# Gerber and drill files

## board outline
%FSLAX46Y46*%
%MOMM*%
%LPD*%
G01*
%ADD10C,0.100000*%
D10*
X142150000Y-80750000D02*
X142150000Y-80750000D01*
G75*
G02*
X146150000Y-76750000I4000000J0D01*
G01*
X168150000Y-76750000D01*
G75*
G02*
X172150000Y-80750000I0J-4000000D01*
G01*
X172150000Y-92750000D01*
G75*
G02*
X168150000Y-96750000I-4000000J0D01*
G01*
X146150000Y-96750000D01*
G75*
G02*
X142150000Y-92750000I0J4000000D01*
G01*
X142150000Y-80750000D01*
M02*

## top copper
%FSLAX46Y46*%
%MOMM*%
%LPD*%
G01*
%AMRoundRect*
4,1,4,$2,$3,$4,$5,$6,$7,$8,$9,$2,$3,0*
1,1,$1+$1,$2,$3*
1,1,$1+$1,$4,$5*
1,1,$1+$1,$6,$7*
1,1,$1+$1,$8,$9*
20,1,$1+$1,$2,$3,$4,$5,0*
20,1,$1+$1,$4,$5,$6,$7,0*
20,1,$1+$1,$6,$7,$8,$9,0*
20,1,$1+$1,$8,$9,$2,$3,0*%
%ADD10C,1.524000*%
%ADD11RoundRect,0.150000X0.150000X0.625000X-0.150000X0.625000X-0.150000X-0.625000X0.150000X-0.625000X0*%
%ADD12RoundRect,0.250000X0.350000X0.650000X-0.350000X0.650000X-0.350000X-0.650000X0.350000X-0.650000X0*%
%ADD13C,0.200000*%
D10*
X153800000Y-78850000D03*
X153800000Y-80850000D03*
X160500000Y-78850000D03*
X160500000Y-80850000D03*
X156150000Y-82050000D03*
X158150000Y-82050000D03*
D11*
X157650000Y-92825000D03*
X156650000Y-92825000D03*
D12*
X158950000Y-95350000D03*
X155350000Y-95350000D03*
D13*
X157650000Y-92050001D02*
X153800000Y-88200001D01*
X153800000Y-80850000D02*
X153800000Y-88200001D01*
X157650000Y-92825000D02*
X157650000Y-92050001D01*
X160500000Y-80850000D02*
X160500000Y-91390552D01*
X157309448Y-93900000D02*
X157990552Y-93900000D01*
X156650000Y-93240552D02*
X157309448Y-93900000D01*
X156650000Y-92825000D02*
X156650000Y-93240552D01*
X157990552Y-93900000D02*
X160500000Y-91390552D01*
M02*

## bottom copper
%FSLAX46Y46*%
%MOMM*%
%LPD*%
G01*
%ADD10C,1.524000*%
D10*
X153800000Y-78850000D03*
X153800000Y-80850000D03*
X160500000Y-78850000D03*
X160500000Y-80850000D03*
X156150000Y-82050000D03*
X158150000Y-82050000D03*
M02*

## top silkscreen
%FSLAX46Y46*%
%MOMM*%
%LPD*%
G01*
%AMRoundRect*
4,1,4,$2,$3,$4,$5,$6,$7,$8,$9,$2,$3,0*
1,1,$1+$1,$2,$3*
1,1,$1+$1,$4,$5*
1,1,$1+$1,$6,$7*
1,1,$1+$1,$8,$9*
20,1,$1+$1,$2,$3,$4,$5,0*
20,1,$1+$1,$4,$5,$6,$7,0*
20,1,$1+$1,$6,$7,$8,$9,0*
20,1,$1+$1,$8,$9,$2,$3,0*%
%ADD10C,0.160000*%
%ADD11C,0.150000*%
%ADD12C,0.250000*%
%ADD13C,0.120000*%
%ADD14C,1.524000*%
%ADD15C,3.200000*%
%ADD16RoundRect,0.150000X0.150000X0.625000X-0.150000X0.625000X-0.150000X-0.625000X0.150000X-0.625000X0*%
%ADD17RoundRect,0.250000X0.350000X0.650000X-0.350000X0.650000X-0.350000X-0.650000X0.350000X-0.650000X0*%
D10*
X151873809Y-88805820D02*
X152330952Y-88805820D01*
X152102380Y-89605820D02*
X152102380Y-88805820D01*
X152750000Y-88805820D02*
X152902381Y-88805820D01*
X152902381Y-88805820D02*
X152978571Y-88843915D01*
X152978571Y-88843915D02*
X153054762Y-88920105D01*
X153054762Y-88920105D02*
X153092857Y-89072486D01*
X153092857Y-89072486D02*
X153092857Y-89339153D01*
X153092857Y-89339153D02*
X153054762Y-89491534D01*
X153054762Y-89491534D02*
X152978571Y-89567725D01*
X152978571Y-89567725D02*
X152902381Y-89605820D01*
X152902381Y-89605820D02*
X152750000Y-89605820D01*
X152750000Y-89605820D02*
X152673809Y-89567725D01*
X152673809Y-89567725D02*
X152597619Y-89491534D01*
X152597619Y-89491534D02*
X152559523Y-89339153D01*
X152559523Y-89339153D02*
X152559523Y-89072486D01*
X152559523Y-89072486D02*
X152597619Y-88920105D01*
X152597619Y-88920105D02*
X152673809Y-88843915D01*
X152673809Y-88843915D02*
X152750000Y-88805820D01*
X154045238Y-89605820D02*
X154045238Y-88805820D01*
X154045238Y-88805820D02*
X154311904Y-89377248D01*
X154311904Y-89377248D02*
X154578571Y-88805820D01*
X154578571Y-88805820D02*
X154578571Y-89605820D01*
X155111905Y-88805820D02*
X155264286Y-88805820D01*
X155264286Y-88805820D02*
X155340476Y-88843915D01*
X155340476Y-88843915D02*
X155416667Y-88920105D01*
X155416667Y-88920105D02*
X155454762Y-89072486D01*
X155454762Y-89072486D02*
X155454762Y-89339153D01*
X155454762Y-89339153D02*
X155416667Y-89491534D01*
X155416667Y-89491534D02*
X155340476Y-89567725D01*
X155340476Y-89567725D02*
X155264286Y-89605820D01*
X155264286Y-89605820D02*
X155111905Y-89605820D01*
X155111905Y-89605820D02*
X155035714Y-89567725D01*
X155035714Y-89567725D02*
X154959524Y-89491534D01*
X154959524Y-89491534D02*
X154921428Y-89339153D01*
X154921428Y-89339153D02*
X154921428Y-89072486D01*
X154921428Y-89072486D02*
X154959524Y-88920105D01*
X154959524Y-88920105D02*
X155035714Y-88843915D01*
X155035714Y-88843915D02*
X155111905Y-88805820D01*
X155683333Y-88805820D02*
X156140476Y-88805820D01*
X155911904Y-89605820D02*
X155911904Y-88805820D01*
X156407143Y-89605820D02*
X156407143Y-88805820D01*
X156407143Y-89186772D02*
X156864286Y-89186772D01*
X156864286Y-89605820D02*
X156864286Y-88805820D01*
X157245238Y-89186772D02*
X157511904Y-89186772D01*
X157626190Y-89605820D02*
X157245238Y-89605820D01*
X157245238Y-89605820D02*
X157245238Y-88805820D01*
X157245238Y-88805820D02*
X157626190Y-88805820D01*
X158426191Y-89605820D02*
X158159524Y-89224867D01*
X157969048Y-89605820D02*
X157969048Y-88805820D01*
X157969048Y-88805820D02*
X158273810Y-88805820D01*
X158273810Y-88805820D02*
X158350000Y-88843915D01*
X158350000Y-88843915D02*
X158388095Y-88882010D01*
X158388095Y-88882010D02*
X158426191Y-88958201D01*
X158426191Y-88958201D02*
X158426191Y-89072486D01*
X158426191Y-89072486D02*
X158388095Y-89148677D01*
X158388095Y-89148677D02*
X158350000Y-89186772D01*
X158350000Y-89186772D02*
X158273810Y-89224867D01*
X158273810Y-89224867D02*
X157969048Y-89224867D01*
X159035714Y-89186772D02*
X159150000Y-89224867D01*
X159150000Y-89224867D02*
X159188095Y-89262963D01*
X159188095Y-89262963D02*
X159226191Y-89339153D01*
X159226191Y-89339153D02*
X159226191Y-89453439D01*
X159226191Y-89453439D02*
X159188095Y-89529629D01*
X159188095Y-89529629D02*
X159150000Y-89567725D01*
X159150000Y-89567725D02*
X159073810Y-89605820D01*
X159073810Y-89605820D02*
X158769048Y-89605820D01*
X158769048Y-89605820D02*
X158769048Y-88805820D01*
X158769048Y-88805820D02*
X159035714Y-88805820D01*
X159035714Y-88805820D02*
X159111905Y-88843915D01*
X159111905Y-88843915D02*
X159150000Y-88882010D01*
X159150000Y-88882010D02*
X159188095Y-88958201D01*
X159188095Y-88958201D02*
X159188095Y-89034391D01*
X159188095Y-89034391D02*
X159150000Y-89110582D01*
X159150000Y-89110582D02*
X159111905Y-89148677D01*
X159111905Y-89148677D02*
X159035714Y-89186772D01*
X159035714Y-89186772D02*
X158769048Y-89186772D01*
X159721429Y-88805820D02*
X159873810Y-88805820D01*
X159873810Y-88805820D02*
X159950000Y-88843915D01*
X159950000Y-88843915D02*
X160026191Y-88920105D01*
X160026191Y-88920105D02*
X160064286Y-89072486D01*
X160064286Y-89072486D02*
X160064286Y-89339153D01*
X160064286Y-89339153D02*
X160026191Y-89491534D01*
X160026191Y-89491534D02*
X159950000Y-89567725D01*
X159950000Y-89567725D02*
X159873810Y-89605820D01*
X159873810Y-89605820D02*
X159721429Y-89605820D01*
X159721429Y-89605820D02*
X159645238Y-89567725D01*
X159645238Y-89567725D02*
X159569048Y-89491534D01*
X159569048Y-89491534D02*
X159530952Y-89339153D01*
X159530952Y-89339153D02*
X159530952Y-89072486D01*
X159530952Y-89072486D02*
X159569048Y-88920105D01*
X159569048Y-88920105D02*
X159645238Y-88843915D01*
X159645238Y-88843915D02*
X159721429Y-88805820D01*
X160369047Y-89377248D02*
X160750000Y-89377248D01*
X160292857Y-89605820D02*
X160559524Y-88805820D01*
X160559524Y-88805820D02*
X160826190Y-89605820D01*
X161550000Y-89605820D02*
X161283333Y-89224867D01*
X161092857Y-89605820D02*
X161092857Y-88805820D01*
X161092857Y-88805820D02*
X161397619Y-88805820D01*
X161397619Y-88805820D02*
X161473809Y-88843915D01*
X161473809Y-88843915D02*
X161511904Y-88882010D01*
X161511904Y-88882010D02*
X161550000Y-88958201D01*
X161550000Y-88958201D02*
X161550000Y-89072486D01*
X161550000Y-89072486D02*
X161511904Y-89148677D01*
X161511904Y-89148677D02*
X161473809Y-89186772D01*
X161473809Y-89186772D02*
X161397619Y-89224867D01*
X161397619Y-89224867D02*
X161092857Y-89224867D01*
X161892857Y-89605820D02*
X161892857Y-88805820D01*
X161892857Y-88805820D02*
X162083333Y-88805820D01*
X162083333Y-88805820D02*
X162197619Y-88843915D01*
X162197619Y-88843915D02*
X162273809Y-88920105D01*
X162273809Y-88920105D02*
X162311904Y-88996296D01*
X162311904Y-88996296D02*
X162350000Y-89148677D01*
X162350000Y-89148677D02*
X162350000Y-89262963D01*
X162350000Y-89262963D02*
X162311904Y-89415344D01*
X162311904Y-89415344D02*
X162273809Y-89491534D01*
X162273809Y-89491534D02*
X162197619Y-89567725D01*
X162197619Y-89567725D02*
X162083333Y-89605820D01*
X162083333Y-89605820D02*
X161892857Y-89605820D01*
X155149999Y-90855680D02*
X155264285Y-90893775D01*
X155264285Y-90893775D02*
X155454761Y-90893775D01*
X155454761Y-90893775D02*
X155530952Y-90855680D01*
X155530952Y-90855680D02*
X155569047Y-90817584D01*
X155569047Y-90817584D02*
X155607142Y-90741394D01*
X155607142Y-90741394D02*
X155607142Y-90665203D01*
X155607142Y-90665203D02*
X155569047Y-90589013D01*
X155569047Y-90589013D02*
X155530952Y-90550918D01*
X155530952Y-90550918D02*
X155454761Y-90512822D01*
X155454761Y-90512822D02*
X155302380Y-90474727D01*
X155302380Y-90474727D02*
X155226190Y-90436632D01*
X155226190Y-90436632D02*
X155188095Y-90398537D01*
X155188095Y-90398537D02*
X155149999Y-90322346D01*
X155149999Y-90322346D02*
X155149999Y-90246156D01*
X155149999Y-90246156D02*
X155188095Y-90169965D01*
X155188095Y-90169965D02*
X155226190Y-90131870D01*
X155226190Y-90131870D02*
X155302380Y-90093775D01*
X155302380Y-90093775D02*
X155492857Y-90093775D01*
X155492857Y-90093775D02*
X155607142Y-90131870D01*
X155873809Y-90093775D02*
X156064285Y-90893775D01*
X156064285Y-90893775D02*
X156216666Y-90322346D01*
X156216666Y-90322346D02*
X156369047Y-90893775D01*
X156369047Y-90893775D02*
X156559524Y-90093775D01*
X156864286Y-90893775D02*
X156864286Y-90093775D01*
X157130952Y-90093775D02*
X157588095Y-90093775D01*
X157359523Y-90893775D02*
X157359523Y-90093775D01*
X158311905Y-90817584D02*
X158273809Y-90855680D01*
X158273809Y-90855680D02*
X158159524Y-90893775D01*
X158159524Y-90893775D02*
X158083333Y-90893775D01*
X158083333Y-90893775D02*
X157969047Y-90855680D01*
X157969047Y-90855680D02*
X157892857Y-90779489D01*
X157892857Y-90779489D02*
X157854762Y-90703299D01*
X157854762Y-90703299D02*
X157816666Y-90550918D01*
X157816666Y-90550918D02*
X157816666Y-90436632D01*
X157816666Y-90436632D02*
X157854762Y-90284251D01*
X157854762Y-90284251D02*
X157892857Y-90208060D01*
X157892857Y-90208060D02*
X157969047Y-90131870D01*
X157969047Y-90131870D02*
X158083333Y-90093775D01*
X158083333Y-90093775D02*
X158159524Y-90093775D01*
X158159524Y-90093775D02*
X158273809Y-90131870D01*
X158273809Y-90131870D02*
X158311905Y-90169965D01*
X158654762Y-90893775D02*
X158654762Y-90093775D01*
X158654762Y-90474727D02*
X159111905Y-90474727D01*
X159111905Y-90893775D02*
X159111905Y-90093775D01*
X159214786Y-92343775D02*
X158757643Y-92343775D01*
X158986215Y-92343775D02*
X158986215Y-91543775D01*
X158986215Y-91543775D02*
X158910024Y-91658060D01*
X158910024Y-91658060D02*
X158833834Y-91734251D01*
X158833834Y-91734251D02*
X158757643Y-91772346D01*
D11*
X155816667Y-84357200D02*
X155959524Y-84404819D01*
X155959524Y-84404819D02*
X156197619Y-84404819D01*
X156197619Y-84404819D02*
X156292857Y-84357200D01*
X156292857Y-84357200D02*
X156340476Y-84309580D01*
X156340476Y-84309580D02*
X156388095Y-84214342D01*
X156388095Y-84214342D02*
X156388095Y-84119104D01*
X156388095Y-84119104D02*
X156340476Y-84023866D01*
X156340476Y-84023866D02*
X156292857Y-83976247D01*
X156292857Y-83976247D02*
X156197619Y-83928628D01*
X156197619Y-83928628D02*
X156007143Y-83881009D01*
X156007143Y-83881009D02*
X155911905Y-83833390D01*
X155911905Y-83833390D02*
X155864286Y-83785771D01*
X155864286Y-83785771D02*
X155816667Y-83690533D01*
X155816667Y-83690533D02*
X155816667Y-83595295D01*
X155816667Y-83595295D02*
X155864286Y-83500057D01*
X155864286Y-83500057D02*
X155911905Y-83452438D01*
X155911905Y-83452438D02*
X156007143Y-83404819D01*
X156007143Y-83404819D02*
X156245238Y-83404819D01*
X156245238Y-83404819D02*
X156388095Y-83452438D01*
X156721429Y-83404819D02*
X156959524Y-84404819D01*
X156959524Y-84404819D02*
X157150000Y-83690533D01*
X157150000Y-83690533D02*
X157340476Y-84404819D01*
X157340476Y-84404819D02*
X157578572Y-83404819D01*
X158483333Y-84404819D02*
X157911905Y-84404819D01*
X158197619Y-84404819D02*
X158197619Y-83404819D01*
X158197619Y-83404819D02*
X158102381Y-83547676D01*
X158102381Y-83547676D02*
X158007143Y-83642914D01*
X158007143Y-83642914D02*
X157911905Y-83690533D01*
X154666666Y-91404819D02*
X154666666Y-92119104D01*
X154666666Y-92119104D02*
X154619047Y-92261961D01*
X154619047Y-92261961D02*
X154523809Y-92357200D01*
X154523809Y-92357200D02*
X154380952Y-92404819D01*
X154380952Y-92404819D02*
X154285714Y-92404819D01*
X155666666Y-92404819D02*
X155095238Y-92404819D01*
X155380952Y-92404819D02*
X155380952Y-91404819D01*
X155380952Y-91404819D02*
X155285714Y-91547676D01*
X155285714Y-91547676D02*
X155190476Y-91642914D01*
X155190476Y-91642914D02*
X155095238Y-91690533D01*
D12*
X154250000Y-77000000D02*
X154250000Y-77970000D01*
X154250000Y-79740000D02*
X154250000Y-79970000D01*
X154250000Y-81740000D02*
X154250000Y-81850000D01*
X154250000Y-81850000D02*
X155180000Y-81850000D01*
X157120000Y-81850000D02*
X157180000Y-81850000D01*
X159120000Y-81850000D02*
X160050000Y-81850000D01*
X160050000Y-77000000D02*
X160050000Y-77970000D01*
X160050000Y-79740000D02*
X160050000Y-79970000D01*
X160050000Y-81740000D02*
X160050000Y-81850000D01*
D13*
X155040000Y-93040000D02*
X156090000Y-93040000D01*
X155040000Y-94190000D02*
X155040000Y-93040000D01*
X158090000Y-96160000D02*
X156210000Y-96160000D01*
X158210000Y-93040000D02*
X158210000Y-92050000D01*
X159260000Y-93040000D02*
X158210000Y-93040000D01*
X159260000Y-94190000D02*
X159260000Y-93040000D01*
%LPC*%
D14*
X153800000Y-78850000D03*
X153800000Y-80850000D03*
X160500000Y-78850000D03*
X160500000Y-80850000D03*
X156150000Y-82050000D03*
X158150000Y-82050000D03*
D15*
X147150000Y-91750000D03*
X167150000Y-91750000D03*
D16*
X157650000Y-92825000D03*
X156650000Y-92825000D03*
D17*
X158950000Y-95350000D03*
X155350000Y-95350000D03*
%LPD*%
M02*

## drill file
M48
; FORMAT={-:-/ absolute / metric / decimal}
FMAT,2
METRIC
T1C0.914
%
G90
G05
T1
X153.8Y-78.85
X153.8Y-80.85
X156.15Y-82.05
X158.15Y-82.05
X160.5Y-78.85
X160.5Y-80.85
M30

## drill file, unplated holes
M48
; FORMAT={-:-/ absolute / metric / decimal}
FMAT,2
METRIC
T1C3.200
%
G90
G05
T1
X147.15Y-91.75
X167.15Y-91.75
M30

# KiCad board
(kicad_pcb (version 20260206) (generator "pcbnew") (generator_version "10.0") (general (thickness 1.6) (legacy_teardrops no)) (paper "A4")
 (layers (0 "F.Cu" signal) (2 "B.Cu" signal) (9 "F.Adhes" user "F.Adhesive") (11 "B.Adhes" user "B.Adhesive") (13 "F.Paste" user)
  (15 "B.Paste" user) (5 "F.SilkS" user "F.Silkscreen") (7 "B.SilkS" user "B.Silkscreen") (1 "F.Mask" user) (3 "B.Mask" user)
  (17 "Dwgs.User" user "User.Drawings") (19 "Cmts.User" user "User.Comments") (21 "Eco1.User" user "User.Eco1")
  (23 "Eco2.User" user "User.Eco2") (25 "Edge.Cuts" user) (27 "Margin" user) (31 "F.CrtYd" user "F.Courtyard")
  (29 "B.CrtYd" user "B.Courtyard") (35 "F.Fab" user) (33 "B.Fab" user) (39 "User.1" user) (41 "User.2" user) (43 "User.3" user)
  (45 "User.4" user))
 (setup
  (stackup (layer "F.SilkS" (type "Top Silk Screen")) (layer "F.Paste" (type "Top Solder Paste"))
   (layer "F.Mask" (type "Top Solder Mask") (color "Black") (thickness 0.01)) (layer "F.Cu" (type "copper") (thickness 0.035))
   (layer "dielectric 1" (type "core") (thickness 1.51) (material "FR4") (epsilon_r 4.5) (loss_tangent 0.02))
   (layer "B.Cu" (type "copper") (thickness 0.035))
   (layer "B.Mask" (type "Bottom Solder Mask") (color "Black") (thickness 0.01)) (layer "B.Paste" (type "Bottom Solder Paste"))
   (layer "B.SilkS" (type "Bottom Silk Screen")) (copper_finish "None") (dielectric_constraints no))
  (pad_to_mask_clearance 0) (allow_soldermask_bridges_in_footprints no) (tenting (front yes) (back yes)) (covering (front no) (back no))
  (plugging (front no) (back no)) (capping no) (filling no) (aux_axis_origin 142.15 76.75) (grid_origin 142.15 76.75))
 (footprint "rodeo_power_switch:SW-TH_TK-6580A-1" (layer "F.Cu") (at 157.15 80.45 180)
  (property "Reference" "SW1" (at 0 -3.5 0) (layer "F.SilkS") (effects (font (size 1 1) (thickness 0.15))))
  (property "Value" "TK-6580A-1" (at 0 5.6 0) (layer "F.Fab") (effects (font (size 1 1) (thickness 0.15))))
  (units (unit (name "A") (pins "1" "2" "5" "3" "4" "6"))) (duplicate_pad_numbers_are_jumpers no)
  (fp_line (start 2.9 3.45) (end 2.9 2.48) (stroke (width 0.25) (type solid)) (layer "F.SilkS"))
  (fp_line (start 2.9 0.71) (end 2.9 0.48) (stroke (width 0.25) (type solid)) (layer "F.SilkS"))
  (fp_line (start 2.9 -1.29) (end 2.9 -1.4) (stroke (width 0.25) (type solid)) (layer "F.SilkS"))
  (fp_line (start 2.9 -1.4) (end 1.97 -1.4) (stroke (width 0.25) (type solid)) (layer "F.SilkS"))
  (fp_line (start 0.03 -1.4) (end -0.03 -1.4) (stroke (width 0.25) (type solid)) (layer "F.SilkS"))
  (fp_line (start -1.97 -1.4) (end -2.9 -1.4) (stroke (width 0.25) (type solid)) (layer "F.SilkS"))
  (fp_line (start -2.9 3.45) (end -2.9 2.48) (stroke (width 0.25) (type solid)) (layer "F.SilkS"))
  (fp_line (start -2.9 0.71) (end -2.9 0.48) (stroke (width 0.25) (type solid)) (layer "F.SilkS"))
  (fp_line (start -2.9 -1.29) (end -2.9 -1.4) (stroke (width 0.25) (type solid)) (layer "F.SilkS"))
  (pad "1" thru_hole circle (at 3.35 1.6) (size 1.524 1.524) (drill 0.9144) (layers "*.Cu" "*.Mask") (remove_unused_layers no)
   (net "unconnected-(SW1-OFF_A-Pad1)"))
  (pad "2" thru_hole circle (at 3.35 -0.4) (size 1.524 1.524) (drill 0.9144) (layers "*.Cu" "*.Mask") (remove_unused_layers no) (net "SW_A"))
  (pad "3" thru_hole circle (at -3.35 1.6) (size 1.524 1.524) (drill 0.9144) (layers "*.Cu" "*.Mask") (remove_unused_layers no)
   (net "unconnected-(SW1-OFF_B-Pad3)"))
  (pad "4" thru_hole circle (at -3.35 -0.4) (size 1.524 1.524) (drill 0.9144) (layers "*.Cu" "*.Mask") (remove_unused_layers no)
   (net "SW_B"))
  (pad "5" thru_hole circle (at 1 -1.6) (size 1.524 1.524) (drill 0.9144) (layers "*.Cu" "*.Mask") (remove_unused_layers no)
   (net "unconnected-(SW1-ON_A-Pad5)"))
  (pad "6" thru_hole circle (at -1 -1.6) (size 1.524 1.524) (drill 0.9144) (layers "*.Cu" "*.Mask") (remove_unused_layers no)
   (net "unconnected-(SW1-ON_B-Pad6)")))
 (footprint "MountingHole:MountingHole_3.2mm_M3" (layer "F.Cu") (at 147.15 91.75)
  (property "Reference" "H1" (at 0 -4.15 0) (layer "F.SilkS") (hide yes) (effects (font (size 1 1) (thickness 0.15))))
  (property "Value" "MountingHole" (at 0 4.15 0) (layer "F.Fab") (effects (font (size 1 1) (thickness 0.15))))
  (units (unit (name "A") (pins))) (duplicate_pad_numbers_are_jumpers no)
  (pad "" np_thru_hole circle (at 0 0) (size 3.2 3.2) (drill 3.2) (layers "*.Cu" "*.Mask")))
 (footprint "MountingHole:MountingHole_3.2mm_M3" (layer "F.Cu") (at 167.15 91.75)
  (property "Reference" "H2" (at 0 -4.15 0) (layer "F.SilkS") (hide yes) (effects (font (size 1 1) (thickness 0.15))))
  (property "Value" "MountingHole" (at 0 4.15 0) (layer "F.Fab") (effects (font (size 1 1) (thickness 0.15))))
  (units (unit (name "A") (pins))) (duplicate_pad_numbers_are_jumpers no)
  (pad "" np_thru_hole circle (at 0 0) (size 3.2 3.2) (drill 3.2) (layers "*.Cu" "*.Mask")))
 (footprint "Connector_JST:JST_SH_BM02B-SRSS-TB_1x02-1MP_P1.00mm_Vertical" (layer "F.Cu") (at 157.15 94.15 180)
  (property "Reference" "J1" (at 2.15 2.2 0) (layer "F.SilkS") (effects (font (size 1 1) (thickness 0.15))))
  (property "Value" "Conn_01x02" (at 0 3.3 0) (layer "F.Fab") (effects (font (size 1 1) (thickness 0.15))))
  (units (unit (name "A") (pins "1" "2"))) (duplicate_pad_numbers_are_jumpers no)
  (fp_line (start 2.11 1.11) (end 1.06 1.11) (stroke (width 0.12) (type solid)) (layer "F.SilkS"))
  (fp_line (start 2.11 -0.04) (end 2.11 1.11) (stroke (width 0.12) (type solid)) (layer "F.SilkS"))
  (fp_line (start -0.94 -2.01) (end 0.94 -2.01) (stroke (width 0.12) (type solid)) (layer "F.SilkS"))
  (fp_line (start -1.06 1.11) (end -1.06 2.1) (stroke (width 0.12) (type solid)) (layer "F.SilkS"))
  (fp_line (start -2.11 1.11) (end -1.06 1.11) (stroke (width 0.12) (type solid)) (layer "F.SilkS"))
  (fp_line (start -2.11 -0.04) (end -2.11 1.11) (stroke (width 0.12) (type solid)) (layer "F.SilkS"))
  (pad "1" smd roundrect (at -0.5 1.325 180) (size 0.6 1.55) (layers "F.Cu" "F.Mask" "F.Paste") (roundrect_rratio 0.25) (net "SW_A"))
  (pad "2" smd roundrect (at 0.5 1.325 180) (size 0.6 1.55) (layers "F.Cu" "F.Mask" "F.Paste") (roundrect_rratio 0.25) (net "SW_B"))
  (pad "MP" smd roundrect (at -1.8 -1.2 180) (size 1.2 1.8) (layers "F.Cu" "F.Mask" "F.Paste") (roundrect_rratio 0.208333))
  (pad "MP" smd roundrect (at 1.8 -1.2 180) (size 1.2 1.8) (layers "F.Cu" "F.Mask" "F.Paste") (roundrect_rratio 0.208333)))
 (gr_rect (start 142.15 76.75) (end 172.15 96.75) (radius 4) (stroke (width 0.1) (type solid)) (fill no) (layer "Edge.Cuts"))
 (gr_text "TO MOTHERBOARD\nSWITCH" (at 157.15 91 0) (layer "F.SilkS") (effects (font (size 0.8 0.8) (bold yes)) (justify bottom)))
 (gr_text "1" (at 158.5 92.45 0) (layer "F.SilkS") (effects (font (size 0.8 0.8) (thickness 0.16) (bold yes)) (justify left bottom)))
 (segment (start 157.65 92.050001) (end 153.8 88.200001) (width 0.2) (layer "F.Cu") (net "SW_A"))
 (segment (start 153.8 80.85) (end 153.8 88.200001) (width 0.2) (layer "F.Cu") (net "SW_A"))
 (segment (start 157.65 92.825) (end 157.65 92.050001) (width 0.2) (layer "F.Cu") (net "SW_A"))
 (segment (start 160.5 80.85) (end 160.5 91.390552) (width 0.2) (layer "F.Cu") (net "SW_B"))
 (segment (start 157.309448 93.9) (end 157.990552 93.9) (width 0.2) (layer "F.Cu") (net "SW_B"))
 (segment (start 156.65 93.240552) (end 157.309448 93.9) (width 0.2) (layer "F.Cu") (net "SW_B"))
 (segment (start 156.65 92.825) (end 156.65 93.240552) (width 0.2) (layer "F.Cu") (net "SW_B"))
 (segment (start 157.990552 93.9) (end 160.5 91.390552) (width 0.2) (layer "F.Cu") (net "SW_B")))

